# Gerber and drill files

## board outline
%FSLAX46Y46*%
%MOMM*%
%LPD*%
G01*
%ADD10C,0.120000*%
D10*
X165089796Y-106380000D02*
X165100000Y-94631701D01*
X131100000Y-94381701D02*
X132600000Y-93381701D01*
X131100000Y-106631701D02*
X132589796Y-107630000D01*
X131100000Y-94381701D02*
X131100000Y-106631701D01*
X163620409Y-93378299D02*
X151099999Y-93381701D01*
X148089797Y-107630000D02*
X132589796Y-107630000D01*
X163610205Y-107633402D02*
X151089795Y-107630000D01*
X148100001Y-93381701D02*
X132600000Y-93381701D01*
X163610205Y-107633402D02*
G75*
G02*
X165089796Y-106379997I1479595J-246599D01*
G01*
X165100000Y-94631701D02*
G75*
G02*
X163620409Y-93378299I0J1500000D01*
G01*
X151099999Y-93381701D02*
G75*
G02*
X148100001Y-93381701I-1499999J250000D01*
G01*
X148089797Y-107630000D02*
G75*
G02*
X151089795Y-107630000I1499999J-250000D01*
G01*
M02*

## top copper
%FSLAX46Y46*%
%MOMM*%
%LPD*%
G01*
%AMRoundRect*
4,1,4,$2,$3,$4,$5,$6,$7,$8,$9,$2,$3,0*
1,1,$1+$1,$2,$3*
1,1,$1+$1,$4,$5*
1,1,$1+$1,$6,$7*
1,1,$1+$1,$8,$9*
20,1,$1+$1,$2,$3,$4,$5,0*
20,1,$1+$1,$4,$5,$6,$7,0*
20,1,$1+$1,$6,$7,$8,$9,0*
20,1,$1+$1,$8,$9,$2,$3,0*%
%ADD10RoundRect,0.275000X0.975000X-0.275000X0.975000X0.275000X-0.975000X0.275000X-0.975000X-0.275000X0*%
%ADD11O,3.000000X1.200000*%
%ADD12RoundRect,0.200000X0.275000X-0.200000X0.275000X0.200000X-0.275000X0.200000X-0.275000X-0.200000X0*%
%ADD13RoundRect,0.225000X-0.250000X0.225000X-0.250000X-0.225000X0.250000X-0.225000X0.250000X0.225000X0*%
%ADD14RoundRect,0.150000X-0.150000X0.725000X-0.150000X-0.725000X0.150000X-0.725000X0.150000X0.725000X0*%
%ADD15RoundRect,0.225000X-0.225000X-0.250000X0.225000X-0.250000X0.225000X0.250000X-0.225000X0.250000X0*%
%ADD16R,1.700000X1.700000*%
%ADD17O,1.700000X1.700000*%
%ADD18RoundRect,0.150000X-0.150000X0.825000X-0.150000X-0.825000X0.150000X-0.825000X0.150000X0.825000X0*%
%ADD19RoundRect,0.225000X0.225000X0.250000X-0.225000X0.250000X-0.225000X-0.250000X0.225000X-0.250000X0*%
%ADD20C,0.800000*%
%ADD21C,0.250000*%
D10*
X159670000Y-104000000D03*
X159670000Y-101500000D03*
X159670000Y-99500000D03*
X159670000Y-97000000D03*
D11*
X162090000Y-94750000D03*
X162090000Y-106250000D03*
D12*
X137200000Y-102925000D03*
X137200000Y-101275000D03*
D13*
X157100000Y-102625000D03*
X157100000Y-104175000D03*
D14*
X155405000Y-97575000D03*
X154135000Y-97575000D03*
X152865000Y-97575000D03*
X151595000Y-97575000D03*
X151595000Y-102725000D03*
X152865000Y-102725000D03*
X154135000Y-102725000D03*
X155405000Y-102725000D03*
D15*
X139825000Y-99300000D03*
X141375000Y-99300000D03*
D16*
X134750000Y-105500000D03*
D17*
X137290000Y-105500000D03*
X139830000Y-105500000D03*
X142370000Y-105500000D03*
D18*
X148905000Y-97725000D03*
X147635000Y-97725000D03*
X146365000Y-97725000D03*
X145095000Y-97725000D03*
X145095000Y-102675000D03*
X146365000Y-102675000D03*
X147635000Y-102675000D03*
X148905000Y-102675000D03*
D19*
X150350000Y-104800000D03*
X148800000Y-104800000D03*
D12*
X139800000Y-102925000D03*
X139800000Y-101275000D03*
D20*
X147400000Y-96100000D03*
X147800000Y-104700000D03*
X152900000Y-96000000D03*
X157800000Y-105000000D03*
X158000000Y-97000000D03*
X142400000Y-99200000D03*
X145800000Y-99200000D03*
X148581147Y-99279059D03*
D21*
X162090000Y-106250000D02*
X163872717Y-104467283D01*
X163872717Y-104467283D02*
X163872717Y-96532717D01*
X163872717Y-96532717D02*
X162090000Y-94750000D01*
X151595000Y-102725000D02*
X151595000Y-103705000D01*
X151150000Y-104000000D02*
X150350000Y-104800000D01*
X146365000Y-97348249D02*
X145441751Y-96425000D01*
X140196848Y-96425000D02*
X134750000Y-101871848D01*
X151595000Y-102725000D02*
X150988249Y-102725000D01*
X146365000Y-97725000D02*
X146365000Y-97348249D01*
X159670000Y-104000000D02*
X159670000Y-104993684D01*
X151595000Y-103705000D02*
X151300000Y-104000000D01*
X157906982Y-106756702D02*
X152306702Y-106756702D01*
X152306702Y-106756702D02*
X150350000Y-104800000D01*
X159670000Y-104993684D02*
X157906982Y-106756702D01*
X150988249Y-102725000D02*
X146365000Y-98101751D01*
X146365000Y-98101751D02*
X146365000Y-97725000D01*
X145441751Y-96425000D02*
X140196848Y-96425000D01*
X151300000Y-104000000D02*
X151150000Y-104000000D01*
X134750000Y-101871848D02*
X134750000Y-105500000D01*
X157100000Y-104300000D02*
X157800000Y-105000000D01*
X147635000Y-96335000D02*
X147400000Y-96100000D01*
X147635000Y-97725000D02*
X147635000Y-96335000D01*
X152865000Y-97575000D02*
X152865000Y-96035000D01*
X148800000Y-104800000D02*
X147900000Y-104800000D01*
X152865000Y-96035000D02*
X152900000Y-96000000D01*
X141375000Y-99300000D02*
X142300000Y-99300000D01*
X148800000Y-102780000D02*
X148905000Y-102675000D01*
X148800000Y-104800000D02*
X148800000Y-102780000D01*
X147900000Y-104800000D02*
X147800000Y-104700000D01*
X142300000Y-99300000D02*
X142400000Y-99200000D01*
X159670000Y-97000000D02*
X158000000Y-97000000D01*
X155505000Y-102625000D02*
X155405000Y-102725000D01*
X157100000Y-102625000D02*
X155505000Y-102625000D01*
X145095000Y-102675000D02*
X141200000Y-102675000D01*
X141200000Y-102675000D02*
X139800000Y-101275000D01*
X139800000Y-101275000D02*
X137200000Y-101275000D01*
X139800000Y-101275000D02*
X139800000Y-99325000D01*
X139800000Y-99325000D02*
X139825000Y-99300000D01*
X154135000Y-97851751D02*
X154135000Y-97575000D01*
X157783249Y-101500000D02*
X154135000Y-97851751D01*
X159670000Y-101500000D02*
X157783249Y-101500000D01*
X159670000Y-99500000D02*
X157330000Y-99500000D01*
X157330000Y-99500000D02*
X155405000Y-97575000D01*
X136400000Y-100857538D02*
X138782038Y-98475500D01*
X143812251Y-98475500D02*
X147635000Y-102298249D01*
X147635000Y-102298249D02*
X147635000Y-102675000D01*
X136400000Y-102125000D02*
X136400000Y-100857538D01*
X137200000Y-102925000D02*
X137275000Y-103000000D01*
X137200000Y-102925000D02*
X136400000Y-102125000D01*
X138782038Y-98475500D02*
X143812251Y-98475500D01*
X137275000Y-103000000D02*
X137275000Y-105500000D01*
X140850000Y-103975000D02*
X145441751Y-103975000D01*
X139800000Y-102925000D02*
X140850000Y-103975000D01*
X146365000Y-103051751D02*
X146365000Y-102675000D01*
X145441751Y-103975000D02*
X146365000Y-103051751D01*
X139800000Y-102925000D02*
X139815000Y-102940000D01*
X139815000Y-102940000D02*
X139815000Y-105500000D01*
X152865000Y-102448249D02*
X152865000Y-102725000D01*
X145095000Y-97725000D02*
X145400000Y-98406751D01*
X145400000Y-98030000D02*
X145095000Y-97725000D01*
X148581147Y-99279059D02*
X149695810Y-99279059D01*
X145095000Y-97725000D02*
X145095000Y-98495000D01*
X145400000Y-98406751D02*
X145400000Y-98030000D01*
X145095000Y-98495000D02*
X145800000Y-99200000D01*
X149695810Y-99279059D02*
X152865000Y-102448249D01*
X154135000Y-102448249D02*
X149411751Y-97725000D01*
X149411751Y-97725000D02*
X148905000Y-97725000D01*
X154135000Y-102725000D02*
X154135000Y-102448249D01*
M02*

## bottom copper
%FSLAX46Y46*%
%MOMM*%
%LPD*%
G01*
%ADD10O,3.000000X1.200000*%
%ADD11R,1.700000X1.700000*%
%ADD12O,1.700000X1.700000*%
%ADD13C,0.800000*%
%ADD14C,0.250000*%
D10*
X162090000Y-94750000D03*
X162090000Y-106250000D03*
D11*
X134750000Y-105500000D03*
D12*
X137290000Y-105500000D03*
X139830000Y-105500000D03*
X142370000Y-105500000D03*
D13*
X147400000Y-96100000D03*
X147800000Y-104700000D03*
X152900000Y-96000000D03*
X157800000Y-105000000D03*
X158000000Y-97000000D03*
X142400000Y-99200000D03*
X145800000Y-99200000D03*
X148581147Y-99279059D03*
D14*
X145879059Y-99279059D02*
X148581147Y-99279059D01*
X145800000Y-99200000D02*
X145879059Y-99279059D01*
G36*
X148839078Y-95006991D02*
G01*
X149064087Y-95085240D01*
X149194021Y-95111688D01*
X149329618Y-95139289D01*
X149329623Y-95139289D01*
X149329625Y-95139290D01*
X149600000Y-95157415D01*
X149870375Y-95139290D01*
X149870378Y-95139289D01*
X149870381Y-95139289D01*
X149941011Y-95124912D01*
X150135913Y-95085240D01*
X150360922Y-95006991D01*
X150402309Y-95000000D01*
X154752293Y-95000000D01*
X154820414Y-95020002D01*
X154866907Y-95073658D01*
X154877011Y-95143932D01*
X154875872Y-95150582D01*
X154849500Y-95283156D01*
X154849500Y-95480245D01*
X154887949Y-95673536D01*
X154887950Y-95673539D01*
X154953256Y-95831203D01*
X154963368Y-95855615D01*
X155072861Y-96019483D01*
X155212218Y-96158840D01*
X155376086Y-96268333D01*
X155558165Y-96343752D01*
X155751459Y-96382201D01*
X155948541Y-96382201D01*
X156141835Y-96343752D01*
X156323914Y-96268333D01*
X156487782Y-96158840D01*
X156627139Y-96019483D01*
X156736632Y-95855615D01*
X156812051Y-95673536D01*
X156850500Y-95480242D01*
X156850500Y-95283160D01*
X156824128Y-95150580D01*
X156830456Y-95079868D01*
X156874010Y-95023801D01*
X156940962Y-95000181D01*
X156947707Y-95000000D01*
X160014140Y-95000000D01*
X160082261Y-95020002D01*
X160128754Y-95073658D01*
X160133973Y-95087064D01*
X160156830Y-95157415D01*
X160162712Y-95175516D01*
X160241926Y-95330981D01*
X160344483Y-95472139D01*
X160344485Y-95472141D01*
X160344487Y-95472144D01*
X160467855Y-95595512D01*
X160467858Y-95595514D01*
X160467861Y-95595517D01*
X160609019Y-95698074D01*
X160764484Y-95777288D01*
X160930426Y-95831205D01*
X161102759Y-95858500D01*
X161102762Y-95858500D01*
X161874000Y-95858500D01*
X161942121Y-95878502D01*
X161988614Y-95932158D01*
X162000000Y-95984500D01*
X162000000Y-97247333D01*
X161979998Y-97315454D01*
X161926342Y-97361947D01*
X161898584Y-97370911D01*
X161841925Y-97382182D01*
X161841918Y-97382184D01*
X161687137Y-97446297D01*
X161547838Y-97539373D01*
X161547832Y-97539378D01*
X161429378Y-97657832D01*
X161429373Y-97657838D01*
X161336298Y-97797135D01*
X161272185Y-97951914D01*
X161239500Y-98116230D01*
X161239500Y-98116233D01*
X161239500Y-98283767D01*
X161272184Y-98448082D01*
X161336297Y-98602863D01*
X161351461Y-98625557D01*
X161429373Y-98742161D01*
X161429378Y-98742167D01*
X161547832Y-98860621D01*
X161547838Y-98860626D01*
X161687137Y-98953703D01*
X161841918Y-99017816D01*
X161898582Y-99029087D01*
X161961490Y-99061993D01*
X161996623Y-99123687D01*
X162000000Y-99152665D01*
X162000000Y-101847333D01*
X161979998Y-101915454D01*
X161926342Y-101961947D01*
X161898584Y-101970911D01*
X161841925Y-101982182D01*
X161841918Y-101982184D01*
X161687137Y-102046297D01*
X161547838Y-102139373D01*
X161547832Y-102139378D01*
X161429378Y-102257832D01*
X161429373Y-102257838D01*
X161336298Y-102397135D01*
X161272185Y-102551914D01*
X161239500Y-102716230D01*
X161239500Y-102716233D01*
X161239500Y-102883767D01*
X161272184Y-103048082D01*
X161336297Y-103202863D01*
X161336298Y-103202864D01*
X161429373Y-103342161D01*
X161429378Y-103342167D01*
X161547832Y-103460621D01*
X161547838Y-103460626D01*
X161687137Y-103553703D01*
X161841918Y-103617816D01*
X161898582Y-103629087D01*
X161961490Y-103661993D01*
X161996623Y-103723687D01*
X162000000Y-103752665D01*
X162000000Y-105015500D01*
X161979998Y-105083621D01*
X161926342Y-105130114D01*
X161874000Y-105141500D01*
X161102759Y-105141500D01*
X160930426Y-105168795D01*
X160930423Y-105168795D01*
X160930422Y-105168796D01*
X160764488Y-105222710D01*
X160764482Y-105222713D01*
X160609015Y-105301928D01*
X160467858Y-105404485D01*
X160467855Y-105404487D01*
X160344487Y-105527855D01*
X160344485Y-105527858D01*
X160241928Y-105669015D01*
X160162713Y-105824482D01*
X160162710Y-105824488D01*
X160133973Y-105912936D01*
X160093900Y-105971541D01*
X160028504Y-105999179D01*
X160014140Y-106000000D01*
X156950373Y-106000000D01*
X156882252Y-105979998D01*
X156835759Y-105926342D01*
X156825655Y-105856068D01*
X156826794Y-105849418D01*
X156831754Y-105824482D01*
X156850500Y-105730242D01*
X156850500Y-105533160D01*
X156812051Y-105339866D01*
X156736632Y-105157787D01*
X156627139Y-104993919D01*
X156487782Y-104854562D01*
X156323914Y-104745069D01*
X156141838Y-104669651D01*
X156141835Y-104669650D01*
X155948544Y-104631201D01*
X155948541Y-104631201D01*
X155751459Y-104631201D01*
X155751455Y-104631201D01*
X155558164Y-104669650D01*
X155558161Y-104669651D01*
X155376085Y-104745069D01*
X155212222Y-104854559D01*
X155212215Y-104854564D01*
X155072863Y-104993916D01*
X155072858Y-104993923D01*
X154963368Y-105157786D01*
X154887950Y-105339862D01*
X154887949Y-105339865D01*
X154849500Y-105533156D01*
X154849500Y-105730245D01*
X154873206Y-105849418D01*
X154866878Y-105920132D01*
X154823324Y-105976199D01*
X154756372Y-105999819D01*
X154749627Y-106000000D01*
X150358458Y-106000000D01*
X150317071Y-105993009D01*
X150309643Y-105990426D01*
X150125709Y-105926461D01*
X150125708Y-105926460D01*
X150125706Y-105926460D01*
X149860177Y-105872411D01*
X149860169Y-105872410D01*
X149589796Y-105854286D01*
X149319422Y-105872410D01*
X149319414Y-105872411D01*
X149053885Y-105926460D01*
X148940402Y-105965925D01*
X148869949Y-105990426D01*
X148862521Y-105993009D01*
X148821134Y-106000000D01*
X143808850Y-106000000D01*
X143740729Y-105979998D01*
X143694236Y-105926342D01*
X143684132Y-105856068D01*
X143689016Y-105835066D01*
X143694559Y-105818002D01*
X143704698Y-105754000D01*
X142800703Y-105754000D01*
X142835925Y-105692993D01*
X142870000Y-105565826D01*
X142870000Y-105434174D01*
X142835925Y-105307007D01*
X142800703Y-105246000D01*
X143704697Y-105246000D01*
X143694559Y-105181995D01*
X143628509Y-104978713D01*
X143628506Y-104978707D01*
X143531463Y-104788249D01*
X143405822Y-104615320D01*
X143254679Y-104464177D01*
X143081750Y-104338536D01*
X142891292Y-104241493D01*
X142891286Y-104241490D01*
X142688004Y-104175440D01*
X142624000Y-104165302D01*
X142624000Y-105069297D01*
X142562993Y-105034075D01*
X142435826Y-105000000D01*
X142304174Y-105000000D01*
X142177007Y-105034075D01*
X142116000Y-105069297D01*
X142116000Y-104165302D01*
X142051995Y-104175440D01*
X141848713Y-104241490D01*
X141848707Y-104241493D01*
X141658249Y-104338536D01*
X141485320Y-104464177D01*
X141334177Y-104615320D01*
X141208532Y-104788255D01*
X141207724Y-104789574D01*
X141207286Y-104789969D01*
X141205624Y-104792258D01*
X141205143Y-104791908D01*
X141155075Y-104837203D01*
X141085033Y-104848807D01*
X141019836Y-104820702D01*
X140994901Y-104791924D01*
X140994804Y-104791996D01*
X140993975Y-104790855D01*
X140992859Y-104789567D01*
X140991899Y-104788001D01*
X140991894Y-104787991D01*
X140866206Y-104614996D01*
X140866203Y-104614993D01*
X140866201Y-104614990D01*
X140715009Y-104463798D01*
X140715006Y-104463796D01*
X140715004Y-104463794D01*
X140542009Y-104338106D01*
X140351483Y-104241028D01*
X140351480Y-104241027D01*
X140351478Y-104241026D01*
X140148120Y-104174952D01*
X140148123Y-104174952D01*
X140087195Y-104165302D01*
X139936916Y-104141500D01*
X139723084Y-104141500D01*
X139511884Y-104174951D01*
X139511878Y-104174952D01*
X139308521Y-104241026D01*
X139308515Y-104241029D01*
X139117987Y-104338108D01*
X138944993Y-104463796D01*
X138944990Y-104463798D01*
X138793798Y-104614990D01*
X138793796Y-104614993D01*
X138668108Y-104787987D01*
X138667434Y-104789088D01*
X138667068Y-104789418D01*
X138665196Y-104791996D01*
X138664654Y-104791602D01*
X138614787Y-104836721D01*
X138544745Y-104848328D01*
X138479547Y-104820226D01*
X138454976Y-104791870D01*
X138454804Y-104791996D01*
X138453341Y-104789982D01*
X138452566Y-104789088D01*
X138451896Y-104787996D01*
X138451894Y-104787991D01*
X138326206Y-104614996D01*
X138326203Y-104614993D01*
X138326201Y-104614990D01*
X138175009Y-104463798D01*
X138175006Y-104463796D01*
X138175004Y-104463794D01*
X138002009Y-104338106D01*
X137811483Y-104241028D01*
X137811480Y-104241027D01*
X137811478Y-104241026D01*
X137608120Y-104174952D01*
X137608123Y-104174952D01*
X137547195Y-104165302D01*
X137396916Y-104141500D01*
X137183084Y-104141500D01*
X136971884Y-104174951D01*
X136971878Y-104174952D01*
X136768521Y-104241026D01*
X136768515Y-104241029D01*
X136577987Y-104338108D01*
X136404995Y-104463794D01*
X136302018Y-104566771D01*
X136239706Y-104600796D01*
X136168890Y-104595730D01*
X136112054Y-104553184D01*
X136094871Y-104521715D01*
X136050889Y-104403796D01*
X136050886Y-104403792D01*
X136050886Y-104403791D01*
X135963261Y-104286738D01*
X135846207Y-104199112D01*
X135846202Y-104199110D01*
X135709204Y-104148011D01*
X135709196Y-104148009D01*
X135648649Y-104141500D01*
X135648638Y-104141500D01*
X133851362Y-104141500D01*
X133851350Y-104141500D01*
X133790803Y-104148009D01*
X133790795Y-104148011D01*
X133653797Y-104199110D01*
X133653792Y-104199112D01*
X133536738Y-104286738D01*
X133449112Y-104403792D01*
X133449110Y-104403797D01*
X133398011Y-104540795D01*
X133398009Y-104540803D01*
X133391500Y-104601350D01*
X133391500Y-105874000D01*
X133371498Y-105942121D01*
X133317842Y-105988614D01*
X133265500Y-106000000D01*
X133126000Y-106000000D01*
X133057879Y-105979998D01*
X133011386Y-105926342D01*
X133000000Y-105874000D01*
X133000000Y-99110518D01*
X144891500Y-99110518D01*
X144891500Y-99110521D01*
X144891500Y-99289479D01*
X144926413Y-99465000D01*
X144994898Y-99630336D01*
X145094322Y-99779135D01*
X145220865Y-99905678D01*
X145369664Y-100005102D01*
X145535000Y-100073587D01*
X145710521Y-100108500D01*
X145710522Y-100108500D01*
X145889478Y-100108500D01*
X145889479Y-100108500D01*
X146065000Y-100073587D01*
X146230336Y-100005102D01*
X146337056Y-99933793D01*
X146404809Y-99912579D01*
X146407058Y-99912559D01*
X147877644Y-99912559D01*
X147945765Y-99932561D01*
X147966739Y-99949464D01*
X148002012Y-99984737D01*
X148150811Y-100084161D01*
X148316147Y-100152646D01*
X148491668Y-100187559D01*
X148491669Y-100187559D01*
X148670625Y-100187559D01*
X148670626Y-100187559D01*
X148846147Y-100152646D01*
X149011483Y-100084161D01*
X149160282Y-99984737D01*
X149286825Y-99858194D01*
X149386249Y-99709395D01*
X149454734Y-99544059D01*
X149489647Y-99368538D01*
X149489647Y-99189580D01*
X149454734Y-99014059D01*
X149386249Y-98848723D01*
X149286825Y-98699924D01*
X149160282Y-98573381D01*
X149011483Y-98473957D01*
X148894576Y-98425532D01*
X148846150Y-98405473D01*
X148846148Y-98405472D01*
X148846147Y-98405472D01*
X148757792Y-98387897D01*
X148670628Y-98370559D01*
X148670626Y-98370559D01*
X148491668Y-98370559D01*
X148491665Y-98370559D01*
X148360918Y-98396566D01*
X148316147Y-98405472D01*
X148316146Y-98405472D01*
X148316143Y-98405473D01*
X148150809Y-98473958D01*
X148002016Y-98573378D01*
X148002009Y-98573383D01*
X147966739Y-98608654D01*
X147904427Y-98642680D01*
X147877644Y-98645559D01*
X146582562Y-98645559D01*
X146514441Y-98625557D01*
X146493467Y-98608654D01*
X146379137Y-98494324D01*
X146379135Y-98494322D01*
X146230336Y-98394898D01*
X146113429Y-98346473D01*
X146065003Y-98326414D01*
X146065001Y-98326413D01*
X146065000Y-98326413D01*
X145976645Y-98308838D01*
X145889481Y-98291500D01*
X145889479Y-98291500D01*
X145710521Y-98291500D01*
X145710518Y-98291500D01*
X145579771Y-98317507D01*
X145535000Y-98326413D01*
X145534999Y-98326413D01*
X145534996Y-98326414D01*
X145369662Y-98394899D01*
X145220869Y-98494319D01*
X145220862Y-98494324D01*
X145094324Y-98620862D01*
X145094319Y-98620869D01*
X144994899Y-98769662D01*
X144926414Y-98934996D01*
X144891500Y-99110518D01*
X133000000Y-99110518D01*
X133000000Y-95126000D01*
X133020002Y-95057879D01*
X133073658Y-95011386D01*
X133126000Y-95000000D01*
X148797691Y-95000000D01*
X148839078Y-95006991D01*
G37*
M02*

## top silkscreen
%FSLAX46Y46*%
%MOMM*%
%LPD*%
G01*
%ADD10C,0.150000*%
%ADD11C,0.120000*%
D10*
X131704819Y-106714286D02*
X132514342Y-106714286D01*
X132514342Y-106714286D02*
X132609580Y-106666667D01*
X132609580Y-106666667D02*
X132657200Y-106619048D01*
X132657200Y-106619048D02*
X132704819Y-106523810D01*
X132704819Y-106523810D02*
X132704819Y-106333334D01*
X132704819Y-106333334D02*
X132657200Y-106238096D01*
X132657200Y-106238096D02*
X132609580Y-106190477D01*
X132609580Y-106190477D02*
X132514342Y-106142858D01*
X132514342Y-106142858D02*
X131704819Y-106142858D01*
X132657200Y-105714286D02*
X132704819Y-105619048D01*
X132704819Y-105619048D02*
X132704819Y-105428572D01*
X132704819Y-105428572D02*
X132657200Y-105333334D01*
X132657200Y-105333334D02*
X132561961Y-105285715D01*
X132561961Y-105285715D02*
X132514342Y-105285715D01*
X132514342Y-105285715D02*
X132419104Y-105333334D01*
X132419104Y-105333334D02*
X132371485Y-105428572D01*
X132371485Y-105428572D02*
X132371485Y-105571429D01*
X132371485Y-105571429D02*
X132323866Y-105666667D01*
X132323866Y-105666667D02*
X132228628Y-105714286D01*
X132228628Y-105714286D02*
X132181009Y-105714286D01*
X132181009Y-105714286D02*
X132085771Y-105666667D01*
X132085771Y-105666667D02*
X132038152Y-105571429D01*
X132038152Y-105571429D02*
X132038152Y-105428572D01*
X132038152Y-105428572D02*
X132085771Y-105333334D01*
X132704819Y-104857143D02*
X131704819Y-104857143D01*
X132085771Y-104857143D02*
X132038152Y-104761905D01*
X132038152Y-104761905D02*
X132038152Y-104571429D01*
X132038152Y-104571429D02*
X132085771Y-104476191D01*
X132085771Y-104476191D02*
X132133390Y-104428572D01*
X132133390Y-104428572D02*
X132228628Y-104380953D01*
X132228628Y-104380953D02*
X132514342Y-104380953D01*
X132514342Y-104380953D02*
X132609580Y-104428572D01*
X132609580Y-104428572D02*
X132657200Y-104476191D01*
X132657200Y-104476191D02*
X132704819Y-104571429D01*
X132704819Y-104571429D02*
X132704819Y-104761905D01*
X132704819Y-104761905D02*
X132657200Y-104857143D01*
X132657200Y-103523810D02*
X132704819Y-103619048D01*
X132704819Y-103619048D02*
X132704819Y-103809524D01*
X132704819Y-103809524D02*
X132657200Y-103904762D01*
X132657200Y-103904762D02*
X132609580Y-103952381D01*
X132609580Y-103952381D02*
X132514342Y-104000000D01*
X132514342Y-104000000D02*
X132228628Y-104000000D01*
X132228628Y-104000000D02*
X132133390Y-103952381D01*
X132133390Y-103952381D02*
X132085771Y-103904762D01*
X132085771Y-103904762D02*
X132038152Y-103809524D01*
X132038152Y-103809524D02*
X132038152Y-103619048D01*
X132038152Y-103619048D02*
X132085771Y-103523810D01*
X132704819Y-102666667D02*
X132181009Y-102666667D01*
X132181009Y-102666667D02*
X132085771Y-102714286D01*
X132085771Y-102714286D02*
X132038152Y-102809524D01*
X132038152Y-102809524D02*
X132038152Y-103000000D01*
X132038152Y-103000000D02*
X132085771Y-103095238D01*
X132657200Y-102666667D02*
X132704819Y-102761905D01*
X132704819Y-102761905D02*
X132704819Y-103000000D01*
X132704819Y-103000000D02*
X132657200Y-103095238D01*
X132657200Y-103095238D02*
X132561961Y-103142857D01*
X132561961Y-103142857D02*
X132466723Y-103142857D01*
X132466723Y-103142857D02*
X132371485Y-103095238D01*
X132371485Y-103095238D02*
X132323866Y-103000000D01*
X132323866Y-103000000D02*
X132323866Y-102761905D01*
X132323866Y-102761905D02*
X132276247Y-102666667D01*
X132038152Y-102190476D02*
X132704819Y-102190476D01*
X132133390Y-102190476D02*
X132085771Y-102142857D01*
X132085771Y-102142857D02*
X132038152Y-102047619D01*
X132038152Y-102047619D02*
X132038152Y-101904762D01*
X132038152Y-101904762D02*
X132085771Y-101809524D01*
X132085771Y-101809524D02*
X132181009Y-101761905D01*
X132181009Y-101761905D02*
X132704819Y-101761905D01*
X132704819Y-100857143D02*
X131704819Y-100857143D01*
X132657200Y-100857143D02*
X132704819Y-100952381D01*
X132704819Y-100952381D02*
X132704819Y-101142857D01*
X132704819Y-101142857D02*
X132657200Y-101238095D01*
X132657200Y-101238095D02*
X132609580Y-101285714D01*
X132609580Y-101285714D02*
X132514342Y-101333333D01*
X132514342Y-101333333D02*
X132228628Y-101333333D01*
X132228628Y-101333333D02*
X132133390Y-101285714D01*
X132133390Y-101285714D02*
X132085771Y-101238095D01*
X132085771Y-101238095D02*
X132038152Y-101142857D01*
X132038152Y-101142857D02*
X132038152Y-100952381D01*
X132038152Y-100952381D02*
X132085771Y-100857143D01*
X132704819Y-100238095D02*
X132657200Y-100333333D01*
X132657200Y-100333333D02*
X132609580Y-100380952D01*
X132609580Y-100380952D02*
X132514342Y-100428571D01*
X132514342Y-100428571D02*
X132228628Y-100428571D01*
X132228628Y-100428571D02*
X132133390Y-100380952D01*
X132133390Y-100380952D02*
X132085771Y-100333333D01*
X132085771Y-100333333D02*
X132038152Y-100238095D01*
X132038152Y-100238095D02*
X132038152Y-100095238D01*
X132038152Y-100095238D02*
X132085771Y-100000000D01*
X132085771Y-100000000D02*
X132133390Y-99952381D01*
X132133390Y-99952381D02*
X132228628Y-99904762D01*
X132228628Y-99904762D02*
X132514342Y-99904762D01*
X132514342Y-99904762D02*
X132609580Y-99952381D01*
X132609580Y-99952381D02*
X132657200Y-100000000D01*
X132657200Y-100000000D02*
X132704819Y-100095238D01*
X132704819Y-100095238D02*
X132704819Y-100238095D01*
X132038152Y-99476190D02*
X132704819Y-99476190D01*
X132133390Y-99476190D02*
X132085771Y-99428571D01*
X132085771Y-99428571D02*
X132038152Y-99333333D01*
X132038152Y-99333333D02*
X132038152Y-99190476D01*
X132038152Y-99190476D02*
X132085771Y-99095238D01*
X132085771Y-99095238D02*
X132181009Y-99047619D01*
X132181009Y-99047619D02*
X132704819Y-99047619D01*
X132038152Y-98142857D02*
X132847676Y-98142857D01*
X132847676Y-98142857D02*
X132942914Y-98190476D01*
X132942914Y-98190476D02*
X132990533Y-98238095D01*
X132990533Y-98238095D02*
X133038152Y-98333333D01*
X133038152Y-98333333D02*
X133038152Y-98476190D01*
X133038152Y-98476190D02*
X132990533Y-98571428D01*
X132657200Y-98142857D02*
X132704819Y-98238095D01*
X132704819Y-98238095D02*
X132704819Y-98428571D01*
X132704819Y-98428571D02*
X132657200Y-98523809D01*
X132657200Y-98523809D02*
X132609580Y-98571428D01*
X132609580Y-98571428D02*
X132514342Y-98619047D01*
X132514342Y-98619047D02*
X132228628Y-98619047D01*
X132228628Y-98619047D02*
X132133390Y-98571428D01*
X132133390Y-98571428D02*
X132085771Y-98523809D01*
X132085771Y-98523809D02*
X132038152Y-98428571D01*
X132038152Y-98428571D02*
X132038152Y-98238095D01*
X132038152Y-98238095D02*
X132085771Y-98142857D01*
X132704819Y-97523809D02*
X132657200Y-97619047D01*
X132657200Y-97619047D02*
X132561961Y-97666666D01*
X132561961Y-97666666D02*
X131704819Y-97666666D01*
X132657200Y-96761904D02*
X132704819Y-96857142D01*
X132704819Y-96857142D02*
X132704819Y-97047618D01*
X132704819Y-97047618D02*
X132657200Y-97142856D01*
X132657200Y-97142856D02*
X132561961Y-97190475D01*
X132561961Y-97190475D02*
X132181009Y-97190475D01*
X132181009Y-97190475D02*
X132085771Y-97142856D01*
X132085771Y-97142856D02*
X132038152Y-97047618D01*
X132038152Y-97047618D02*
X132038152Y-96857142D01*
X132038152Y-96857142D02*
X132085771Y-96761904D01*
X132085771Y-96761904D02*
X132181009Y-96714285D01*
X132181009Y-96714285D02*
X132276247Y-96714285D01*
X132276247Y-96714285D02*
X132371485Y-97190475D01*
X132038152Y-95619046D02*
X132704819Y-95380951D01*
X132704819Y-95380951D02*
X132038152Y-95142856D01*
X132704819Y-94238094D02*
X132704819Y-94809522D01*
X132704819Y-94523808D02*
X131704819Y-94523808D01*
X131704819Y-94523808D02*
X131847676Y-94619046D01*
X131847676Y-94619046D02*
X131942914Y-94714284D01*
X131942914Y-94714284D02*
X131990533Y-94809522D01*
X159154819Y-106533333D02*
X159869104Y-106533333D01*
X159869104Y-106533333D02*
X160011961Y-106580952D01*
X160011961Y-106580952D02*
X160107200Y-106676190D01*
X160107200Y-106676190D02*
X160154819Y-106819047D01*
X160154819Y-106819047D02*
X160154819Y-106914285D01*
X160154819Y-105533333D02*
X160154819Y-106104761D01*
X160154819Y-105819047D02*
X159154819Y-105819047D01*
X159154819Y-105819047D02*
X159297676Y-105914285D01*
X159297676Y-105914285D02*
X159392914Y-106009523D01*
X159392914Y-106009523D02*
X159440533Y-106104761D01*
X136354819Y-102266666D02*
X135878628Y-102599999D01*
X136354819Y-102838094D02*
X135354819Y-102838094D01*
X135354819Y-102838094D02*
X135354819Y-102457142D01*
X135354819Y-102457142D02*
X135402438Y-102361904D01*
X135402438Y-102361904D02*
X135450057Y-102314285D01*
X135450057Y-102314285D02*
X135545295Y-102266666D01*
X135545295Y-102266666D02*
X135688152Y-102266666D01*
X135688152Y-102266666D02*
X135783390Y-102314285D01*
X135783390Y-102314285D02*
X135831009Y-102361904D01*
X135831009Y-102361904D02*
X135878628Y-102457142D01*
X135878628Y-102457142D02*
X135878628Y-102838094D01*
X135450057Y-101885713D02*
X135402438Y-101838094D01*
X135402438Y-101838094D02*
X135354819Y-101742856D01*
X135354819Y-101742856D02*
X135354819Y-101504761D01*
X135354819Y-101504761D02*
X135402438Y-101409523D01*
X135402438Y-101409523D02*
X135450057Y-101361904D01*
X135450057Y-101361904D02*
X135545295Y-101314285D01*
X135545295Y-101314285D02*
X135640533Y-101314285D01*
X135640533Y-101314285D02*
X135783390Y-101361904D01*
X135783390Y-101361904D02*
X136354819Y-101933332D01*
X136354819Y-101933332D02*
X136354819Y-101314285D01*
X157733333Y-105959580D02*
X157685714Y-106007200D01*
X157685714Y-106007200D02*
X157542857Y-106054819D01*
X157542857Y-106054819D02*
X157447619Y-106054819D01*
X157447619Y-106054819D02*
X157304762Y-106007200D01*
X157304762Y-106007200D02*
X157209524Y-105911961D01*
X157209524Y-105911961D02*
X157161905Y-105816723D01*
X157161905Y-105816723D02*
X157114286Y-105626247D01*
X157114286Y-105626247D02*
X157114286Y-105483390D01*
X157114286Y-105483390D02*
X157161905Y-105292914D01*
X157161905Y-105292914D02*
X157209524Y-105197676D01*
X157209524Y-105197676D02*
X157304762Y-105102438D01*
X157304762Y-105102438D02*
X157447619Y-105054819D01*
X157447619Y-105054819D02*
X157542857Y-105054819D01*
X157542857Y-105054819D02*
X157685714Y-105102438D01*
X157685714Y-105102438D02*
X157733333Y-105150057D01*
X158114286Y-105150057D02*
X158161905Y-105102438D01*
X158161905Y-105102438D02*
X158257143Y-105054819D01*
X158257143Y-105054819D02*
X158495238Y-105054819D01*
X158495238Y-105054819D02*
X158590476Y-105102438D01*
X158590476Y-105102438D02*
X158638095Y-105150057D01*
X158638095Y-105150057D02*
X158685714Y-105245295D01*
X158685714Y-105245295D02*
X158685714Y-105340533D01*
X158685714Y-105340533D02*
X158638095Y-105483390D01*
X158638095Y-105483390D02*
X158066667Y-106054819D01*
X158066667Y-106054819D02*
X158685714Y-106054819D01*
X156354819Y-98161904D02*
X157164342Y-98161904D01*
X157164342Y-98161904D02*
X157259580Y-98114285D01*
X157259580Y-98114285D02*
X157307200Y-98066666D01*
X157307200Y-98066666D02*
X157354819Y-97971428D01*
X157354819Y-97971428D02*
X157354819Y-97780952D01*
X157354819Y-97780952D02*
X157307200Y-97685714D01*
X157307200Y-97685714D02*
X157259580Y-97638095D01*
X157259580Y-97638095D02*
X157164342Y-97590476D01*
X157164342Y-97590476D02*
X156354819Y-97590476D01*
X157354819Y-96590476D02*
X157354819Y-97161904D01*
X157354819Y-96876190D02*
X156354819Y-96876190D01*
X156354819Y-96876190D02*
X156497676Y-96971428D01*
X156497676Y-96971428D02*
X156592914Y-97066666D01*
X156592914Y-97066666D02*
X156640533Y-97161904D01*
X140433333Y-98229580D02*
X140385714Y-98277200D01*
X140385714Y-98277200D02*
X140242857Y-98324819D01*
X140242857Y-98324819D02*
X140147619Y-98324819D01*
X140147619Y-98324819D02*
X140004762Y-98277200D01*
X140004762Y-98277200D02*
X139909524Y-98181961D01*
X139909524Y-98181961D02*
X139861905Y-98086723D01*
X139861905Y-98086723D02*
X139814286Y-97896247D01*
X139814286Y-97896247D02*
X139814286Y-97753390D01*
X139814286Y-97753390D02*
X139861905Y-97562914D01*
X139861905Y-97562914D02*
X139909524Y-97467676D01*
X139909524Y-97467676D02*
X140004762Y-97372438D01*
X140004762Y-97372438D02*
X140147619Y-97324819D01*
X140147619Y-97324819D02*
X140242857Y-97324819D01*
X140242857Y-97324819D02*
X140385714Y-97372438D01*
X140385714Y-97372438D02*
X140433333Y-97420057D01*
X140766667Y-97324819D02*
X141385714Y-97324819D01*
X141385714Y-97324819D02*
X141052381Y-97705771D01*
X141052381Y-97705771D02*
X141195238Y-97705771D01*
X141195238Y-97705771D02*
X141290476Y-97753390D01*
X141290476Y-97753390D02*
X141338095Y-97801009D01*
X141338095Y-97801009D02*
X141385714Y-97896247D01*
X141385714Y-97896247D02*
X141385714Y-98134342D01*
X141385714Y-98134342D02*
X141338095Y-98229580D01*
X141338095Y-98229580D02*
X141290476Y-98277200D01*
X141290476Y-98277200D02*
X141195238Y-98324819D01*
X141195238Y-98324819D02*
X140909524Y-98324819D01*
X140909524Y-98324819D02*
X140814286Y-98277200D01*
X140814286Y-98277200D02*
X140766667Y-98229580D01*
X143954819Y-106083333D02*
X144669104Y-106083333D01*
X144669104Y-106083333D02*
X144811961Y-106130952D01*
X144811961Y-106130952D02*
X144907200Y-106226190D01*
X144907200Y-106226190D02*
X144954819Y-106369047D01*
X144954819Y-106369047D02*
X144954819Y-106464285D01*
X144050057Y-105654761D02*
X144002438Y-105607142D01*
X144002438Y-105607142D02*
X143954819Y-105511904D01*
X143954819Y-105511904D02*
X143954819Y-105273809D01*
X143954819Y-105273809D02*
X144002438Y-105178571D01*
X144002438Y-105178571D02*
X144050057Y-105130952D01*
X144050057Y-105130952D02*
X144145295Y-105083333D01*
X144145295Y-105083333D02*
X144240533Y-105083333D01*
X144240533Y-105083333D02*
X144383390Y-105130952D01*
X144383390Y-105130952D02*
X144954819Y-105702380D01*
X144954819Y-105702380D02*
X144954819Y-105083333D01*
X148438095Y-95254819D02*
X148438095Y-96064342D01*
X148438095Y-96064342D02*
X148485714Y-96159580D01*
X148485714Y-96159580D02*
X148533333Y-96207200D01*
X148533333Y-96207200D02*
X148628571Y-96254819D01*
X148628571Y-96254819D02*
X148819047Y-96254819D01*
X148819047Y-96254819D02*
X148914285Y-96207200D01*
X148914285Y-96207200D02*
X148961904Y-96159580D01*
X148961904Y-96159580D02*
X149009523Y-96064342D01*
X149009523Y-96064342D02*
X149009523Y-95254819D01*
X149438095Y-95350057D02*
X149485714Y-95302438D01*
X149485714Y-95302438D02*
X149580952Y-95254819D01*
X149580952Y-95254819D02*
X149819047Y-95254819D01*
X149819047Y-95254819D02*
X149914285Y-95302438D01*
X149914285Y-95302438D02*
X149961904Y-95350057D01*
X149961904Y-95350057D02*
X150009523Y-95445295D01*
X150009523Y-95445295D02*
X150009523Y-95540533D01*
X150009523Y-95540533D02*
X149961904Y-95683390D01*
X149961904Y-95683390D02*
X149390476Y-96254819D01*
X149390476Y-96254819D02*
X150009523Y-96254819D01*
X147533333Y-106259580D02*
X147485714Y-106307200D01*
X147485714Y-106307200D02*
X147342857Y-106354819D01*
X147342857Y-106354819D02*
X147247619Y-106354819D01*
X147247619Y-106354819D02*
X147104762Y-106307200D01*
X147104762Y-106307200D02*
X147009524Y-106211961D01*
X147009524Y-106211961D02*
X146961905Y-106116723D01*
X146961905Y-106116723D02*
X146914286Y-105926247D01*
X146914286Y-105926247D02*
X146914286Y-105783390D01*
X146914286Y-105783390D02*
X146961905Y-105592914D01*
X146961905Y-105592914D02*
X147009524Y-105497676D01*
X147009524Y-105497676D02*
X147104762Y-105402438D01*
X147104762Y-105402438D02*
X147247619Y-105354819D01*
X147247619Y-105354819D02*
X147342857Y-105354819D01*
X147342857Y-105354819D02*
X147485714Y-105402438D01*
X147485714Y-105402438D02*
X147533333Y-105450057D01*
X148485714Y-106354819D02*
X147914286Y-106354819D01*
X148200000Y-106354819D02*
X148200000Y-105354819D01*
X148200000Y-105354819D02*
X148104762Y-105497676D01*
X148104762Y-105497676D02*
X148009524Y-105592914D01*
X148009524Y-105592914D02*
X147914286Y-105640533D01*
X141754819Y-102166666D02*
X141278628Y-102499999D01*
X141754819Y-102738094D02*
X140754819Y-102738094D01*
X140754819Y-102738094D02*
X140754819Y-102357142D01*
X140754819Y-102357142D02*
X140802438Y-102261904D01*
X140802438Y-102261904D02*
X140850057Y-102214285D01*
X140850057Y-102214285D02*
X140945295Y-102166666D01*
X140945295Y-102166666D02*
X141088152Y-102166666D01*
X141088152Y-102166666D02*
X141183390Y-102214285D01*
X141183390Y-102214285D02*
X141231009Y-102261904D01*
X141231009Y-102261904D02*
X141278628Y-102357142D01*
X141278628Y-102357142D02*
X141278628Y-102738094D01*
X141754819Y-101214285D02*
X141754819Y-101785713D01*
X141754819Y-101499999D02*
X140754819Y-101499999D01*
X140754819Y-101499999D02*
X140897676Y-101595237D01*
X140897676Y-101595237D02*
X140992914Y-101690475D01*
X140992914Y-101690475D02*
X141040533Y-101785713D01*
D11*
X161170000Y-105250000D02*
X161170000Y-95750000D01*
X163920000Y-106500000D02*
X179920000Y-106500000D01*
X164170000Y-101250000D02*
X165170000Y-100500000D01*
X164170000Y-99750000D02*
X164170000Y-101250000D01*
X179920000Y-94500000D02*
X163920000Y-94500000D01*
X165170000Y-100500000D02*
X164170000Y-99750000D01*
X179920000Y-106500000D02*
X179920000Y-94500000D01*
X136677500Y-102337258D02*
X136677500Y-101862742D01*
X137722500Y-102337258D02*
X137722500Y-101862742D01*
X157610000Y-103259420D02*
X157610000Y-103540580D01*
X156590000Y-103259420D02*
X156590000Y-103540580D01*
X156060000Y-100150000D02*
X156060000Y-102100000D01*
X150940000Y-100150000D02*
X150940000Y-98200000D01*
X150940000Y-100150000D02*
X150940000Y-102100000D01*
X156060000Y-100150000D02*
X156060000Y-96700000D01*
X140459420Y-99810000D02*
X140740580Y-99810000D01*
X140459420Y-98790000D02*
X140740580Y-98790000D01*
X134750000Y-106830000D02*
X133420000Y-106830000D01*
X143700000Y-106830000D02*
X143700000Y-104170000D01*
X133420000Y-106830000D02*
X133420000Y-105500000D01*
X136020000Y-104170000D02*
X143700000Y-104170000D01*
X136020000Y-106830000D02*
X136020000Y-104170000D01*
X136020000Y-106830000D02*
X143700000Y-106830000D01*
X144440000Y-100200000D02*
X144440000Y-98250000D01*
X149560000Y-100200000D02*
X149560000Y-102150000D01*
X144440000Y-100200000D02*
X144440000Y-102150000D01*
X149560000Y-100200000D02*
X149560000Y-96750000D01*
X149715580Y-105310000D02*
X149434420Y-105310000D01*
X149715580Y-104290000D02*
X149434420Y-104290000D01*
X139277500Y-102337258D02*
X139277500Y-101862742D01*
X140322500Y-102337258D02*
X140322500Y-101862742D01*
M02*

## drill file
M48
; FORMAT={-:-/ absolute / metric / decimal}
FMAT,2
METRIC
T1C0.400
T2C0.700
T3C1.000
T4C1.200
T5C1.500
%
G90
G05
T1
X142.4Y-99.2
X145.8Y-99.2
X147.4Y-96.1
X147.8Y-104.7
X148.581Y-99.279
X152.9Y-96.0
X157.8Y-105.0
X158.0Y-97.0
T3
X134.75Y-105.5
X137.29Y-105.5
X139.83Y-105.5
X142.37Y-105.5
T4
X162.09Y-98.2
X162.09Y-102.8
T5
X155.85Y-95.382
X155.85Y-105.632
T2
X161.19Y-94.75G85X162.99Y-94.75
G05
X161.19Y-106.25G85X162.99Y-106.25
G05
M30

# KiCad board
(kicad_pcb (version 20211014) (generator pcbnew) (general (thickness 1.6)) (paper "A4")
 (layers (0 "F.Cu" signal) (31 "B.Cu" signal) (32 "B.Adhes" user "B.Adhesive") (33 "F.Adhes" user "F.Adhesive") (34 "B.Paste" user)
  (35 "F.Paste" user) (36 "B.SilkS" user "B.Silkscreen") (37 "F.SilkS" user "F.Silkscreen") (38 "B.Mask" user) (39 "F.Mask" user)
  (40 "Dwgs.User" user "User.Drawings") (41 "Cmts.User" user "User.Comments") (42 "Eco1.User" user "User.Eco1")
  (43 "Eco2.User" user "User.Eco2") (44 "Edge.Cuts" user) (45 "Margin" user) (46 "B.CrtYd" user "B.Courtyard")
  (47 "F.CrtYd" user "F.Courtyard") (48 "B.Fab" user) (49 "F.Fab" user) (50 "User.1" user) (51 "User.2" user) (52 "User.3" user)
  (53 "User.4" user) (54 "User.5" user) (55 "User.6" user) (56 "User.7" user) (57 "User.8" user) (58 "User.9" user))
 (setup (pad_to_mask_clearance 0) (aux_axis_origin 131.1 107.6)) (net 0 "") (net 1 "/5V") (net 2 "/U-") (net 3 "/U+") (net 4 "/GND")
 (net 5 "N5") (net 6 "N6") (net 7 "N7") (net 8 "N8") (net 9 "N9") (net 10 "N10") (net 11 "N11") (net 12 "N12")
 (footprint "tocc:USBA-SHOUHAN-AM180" (layer "F.Cu") (at 159.67 100.5 90)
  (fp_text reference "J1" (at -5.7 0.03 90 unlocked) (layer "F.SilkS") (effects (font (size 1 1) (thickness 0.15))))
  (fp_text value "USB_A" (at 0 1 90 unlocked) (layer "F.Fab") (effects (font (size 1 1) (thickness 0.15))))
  (fp_line (start -4.75 1.5) (end 4.75 1.5) (layer "F.SilkS") (width 0.12))
  (fp_line (start -6 4.25) (end -6 20.25) (layer "F.SilkS") (width 0.12))
  (fp_line (start -0.75 4.5) (end 0 5.5) (layer "F.SilkS") (width 0.12))
  (fp_line (start 0.75 4.5) (end -0.75 4.5) (layer "F.SilkS") (width 0.12))
  (fp_line (start 6 20.25) (end 6 4.25) (layer "F.SilkS") (width 0.12))
  (fp_line (start 0 5.5) (end 0.75 4.5) (layer "F.SilkS") (width 0.12))
  (fp_line (start -6 20.25) (end 6 20.25) (layer "F.SilkS") (width 0.12))
  (pad "" np_thru_hole circle (at -2.3 2.42 90) (size 1.2 1.2) (drill 1.2) (layers F&B.Cu *.Mask))
  (pad "" np_thru_hole circle (at 2.3 2.42 90) (size 1.2 1.2) (drill 1.2) (layers F&B.Cu *.Mask))
  (pad "1" smd roundrect (at -3.5 0 90) (size 1.1 2.5) (layers "F.Cu" "F.Paste" "F.Mask") (roundrect_rratio 0.25) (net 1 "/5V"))
  (pad "2" smd roundrect (at -1 0 90) (size 1.1 2.5) (layers "F.Cu" "F.Paste" "F.Mask") (roundrect_rratio 0.25) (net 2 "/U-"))
  (pad "3" smd roundrect (at 1 0 90) (size 1.1 2.5) (layers "F.Cu" "F.Paste" "F.Mask") (roundrect_rratio 0.25) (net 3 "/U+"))
  (pad "4" smd roundrect (at 3.5 0 90) (size 1.1 2.5) (layers "F.Cu" "F.Paste" "F.Mask") (roundrect_rratio 0.25) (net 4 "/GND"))
  (pad "5" thru_hole oval (at 5.75 2.42 90) (size 1.2 3) (drill oval 0.7 2.5) (layers *.Cu *.Mask) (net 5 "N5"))
  (pad "5" thru_hole oval (at -5.75 2.42 90) (size 1.2 3) (drill oval 0.7 2.5) (layers *.Cu *.Mask) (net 5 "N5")))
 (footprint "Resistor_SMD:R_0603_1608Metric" (layer "F.Cu") (at 137.2 102.1 90)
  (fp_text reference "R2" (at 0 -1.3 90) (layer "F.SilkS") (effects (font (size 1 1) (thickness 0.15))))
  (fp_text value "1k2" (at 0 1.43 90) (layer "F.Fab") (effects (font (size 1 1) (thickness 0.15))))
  (fp_line (start -0.237258 -0.5225) (end 0.237258 -0.5225) (layer "F.SilkS") (width 0.12))
  (fp_line (start -0.237258 0.5225) (end 0.237258 0.5225) (layer "F.SilkS") (width 0.12))
  (pad "1" smd roundrect (at -0.825 0 90) (size 0.8 0.95) (layers "F.Cu" "F.Paste" "F.Mask") (roundrect_rratio 0.25) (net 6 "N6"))
  (pad "2" smd roundrect (at 0.825 0 90) (size 0.8 0.95) (layers "F.Cu" "F.Paste" "F.Mask") (roundrect_rratio 0.25) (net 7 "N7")))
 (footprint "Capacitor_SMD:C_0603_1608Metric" (layer "F.Cu") (at 157.1 103.4 -90)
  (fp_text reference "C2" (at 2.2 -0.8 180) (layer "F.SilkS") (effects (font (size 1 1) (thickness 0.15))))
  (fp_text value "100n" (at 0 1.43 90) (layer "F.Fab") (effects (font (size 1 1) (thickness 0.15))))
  (fp_line (start -0.14058 -0.51) (end 0.14058 -0.51) (layer "F.SilkS") (width 0.12))
  (fp_line (start -0.14058 0.51) (end 0.14058 0.51) (layer "F.SilkS") (width 0.12))
  (pad "1" smd roundrect (at -0.775 0 270) (size 0.9 0.95) (layers "F.Cu" "F.Paste" "F.Mask") (roundrect_rratio 0.25) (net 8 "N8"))
  (pad "2" smd roundrect (at 0.775 0 270) (size 0.9 0.95) (layers "F.Cu" "F.Paste" "F.Mask") (roundrect_rratio 0.25) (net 4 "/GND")))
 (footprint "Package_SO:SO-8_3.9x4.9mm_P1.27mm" (layer "F.Cu") (at 153.5 100.15 -90)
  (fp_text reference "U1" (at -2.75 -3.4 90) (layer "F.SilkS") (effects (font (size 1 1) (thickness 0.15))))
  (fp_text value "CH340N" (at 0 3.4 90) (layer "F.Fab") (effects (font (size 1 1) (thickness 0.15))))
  (fp_line (start 0 -2.56) (end 1.95 -2.56) (layer "F.SilkS") (width 0.12))
  (fp_line (start 0 2.56) (end -1.95 2.56) (layer "F.SilkS") (width 0.12))
  (fp_line (start 0 2.56) (end 1.95 2.56) (layer "F.SilkS") (width 0.12))
  (fp_line (start 0 -2.56) (end -3.45 -2.56) (layer "F.SilkS") (width 0.12))
  (pad "1" smd roundrect (at -2.575 -1.905 270) (size 1.75 0.6) (layers "F.Cu" "F.Paste" "F.Mask") (roundrect_rratio 0.25) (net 3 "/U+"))
  (pad "2" smd roundrect (at -2.575 -0.635 270) (size 1.75 0.6) (layers "F.Cu" "F.Paste" "F.Mask") (roundrect_rratio 0.25) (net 2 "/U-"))
  (pad "3" smd roundrect (at -2.575 0.635 270) (size 1.75 0.6) (layers "F.Cu" "F.Paste" "F.Mask") (roundrect_rratio 0.25) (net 4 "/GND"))
  (pad "4" smd roundrect (at -2.575 1.905 270) (size 1.75 0.6) (layers "F.Cu" "F.Paste" "F.Mask") (roundrect_rratio 0.25) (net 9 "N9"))
  (pad "5" smd roundrect (at 2.575 1.905 270) (size 1.75 0.6) (layers "F.Cu" "F.Paste" "F.Mask") (roundrect_rratio 0.25) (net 1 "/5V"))
  (pad "6" smd roundrect (at 2.575 0.635 270) (size 1.75 0.6) (layers "F.Cu" "F.Paste" "F.Mask") (roundrect_rratio 0.25) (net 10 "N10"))
  (pad "7" smd roundrect (at 2.575 -0.635 270) (size 1.75 0.6) (layers "F.Cu" "F.Paste" "F.Mask") (roundrect_rratio 0.25) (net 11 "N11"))
  (pad "8" smd roundrect (at 2.575 -1.905 270) (size 1.75 0.6) (layers "F.Cu" "F.Paste" "F.Mask") (roundrect_rratio 0.25) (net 8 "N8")))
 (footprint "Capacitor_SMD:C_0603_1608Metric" (layer "F.Cu") (at 140.6 99.3)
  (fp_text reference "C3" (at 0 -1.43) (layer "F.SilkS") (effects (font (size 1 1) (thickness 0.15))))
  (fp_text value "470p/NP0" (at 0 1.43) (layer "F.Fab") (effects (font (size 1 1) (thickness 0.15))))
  (fp_line (start -0.14058 0.51) (end 0.14058 0.51) (layer "F.SilkS") (width 0.12))
  (fp_line (start -0.14058 -0.51) (end 0.14058 -0.51) (layer "F.SilkS") (width 0.12))
  (pad "1" smd roundrect (at -0.775 0) (size 0.9 0.95) (layers "F.Cu" "F.Paste" "F.Mask") (roundrect_rratio 0.25) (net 7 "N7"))
  (pad "2" smd roundrect (at 0.775 0) (size 0.9 0.95) (layers "F.Cu" "F.Paste" "F.Mask") (roundrect_rratio 0.25) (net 4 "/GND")))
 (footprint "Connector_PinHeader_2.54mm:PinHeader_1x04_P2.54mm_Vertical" (layer "F.Cu") (at 134.75 105.5 90)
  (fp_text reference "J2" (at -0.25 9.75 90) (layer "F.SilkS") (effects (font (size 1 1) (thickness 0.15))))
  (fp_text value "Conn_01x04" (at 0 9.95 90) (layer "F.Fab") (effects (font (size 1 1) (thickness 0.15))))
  (fp_line (start -1.33 0) (end -1.33 -1.33) (layer "F.SilkS") (width 0.12))
  (fp_line (start -1.33 8.95) (end 1.33 8.95) (layer "F.SilkS") (width 0.12))
  (fp_line (start -1.33 -1.33) (end 0 -1.33) (layer "F.SilkS") (width 0.12))
  (fp_line (start 1.33 1.27) (end 1.33 8.95) (layer "F.SilkS") (width 0.12))
  (fp_line (start -1.33 1.27) (end 1.33 1.27) (layer "F.SilkS") (width 0.12))
  (fp_line (start -1.33 1.27) (end -1.33 8.95) (layer "F.SilkS") (width 0.12))
  (pad "1" thru_hole rect (at 0 0 90) (size 1.7 1.7) (drill 1) (layers *.Cu *.Mask) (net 1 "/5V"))
  (pad "2" thru_hole oval (at 0 2.54 90) (size 1.7 1.7) (drill 1) (layers *.Cu *.Mask) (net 6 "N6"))
  (pad "3" thru_hole oval (at 0 5.08 90) (size 1.7 1.7) (drill 1) (layers *.Cu *.Mask) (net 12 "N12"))
  (pad "4" thru_hole oval (at 0 7.62 90) (size 1.7 1.7) (drill 1) (layers *.Cu *.Mask) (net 4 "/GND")))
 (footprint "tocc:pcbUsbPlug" (layer "F.Cu") (at 129.1 107.631701)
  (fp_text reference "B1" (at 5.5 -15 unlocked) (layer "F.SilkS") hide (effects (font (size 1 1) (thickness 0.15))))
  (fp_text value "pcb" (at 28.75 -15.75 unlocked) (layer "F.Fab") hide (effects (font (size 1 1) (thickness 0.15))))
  (fp_line (start 35.989796 -1.251701) (end 36 -13) (layer "Edge.Cuts") (width 0.12))
  (fp_line (start 2 -13.25) (end 3.5 -14.25) (layer "Edge.Cuts") (width 0.12))
  (fp_line (start 2 -1) (end 3.489796 -0.001701) (layer "Edge.Cuts") (width 0.12))
  (fp_line (start 2 -13.25) (end 2 -1) (layer "Edge.Cuts") (width 0.12))
  (fp_line (start 34.520409 -14.253402) (end 21.999999 -14.25) (layer "Edge.Cuts") (width 0.12))
  (fp_line (start 18.989797 -0.001701) (end 3.489796 -0.001701) (layer "Edge.Cuts") (width 0.12))
  (fp_line (start 34.510205 0.001701) (end 21.989795 -0.001701) (layer "Edge.Cuts") (width 0.12))
  (fp_line (start 19.000001 -14.25) (end 3.5 -14.25) (layer "Edge.Cuts") (width 0.12))
  (fp_arc (start 34.510205 0.001701) (mid 35.020233 -0.896232) (end 35.989796 -1.251701) (layer "Edge.Cuts") (width 0.12))
  (fp_arc (start 36 -13) (mid 35.030437 -13.35547) (end 34.520409 -14.253402) (layer "Edge.Cuts") (width 0.12))
  (fp_arc (start 21.999999 -14.25) (mid 20.5 -12.97931) (end 19.000001 -14.25) (layer "Edge.Cuts") (width 0.12))
  (fp_arc (start 18.989797 -0.001701) (mid 20.489796 -1.272391) (end 21.989795 -0.001701) (layer "Edge.Cuts") (width 0.12))
  (pad "" np_thru_hole circle (at 26.75 -12.25) (size 1.5 1.5) (drill 1.5) (layers F&B.Cu *.Mask))
  (pad "" np_thru_hole circle (at 26.75 -2) (size 1.5 1.5) (drill 1.5) (layers F&B.Cu *.Mask)))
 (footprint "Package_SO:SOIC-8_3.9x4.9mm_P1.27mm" (layer "F.Cu") (at 147 100.2 -90)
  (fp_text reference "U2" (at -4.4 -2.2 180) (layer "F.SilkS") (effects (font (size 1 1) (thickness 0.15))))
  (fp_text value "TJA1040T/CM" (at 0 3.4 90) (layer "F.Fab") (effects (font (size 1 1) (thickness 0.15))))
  (fp_line (start 0 2.56) (end -1.95 2.56) (layer "F.SilkS") (width 0.12))
  (fp_line (start 0 -2.56) (end 1.95 -2.56) (layer "F.SilkS") (width 0.12))
  (fp_line (start 0 2.56) (end 1.95 2.56) (layer "F.SilkS") (width 0.12))
  (fp_line (start 0 -2.56) (end -3.45 -2.56) (layer "F.SilkS") (width 0.12))
  (pad "1" smd roundrect (at -2.475 -1.905 270) (size 1.95 0.6) (layers "F.Cu" "F.Paste" "F.Mask") (roundrect_rratio 0.25) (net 11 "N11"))
  (pad "2" smd roundrect (at -2.475 -0.635 270) (size 1.95 0.6) (layers "F.Cu" "F.Paste" "F.Mask") (roundrect_rratio 0.25) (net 4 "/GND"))
  (pad "3" smd roundrect (at -2.475 0.635 270) (size 1.95 0.6) (layers "F.Cu" "F.Paste" "F.Mask") (roundrect_rratio 0.25) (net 1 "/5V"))
  (pad "4" smd roundrect (at -2.475 1.905 270) (size 1.95 0.6) (layers "F.Cu" "F.Paste" "F.Mask") (roundrect_rratio 0.25) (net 10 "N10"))
  (pad "5" smd roundrect (at 2.475 1.905 270) (size 1.95 0.6) (layers "F.Cu" "F.Paste" "F.Mask") (roundrect_rratio 0.25) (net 7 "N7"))
  (pad "6" smd roundrect (at 2.475 0.635 270) (size 1.95 0.6) (layers "F.Cu" "F.Paste" "F.Mask") (roundrect_rratio 0.25) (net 12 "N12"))
  (pad "7" smd roundrect (at 2.475 -0.635 270) (size 1.95 0.6) (layers "F.Cu" "F.Paste" "F.Mask") (roundrect_rratio 0.25) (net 6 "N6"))
  (pad "8" smd roundrect (at 2.475 -1.905 270) (size 1.95 0.6) (layers "F.Cu" "F.Paste" "F.Mask") (roundrect_rratio 0.25) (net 4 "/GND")))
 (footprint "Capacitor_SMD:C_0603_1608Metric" (layer "F.Cu") (at 149.575 104.8 180)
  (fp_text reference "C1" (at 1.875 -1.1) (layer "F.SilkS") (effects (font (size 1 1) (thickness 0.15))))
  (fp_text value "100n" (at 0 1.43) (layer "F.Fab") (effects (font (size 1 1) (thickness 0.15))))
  (fp_line (start -0.14058 -0.51) (end 0.14058 -0.51) (layer "F.SilkS") (width 0.12))
  (fp_line (start -0.14058 0.51) (end 0.14058 0.51) (layer "F.SilkS") (width 0.12))
  (pad "1" smd roundrect (at -0.775 0 180) (size 0.9 0.95) (layers "F.Cu" "F.Paste" "F.Mask") (roundrect_rratio 0.25) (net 1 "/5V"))
  (pad "2" smd roundrect (at 0.775 0 180) (size 0.9 0.95) (layers "F.Cu" "F.Paste" "F.Mask") (roundrect_rratio 0.25) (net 4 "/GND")))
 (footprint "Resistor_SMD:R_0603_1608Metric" (layer "F.Cu") (at 139.8 102.1 90)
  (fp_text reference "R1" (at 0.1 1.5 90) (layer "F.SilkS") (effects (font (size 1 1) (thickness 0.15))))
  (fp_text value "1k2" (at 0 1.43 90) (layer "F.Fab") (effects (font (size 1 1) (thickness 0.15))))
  (fp_line (start -0.237258 -0.5225) (end 0.237258 -0.5225) (layer "F.SilkS") (width 0.12))
  (fp_line (start -0.237258 0.5225) (end 0.237258 0.5225) (layer "F.SilkS") (width 0.12))
  (pad "1" smd roundrect (at -0.825 0 90) (size 0.8 0.95) (layers "F.Cu" "F.Paste" "F.Mask") (roundrect_rratio 0.25) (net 12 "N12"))
  (pad "2" smd roundrect (at 0.825 0 90) (size 0.8 0.95) (layers "F.Cu" "F.Paste" "F.Mask") (roundrect_rratio 0.25) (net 7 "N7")))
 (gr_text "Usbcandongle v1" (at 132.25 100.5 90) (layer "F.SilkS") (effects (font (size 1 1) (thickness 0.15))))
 (segment (start 162.09 106.25) (end 163.872717 104.467283) (width 0.25) (layer "F.Cu") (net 5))
 (segment (start 163.872717 104.467283) (end 163.872717 96.532717) (width 0.25) (layer "F.Cu") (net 5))
 (segment (start 163.872717 96.532717) (end 162.09 94.75) (width 0.25) (layer "F.Cu") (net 5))
 (segment (start 151.595 102.725) (end 151.595 103.705) (width 0.25) (layer "F.Cu") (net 1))
 (segment (start 151.15 104) (end 150.35 104.8) (width 0.25) (layer "F.Cu") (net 1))
 (segment (start 146.365 97.348249) (end 145.441751 96.425) (width 0.25) (layer "F.Cu") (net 1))
 (segment (start 140.196848 96.425) (end 134.75 101.871848) (width 0.25) (layer "F.Cu") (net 1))
 (segment (start 151.595 102.725) (end 150.988249 102.725) (width 0.25) (layer "F.Cu") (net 1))
 (segment (start 146.365 97.725) (end 146.365 97.348249) (width 0.25) (layer "F.Cu") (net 1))
 (segment (start 159.67 104) (end 159.67 104.993684) (width 0.25) (layer "F.Cu") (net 1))
 (segment (start 151.595 103.705) (end 151.3 104) (width 0.25) (layer "F.Cu") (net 1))
 (segment (start 157.906982 106.756702) (end 152.306702 106.756702) (width 0.25) (layer "F.Cu") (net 1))
 (segment (start 152.306702 106.756702) (end 150.35 104.8) (width 0.25) (layer "F.Cu") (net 1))
 (segment (start 159.67 104.993684) (end 157.906982 106.756702) (width 0.25) (layer "F.Cu") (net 1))
 (segment (start 150.988249 102.725) (end 146.365 98.101751) (width 0.25) (layer "F.Cu") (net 1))
 (segment (start 146.365 98.101751) (end 146.365 97.725) (width 0.25) (layer "F.Cu") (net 1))
 (segment (start 145.441751 96.425) (end 140.196848 96.425) (width 0.25) (layer "F.Cu") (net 1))
 (segment (start 151.3 104) (end 151.15 104) (width 0.25) (layer "F.Cu") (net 1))
 (segment (start 134.75 101.871848) (end 134.75 105.5) (width 0.25) (layer "F.Cu") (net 1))
 (segment (start 157.1 104.3) (end 157.8 105) (width 0.25) (layer "F.Cu") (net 4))
 (segment (start 147.635 96.335) (end 147.4 96.1) (width 0.25) (layer "F.Cu") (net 4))
 (segment (start 147.635 97.725) (end 147.635 96.335) (width 0.25) (layer "F.Cu") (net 4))
 (segment (start 152.865 97.575) (end 152.865 96.035) (width 0.25) (layer "F.Cu") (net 4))
 (segment (start 148.8 104.8) (end 147.9 104.8) (width 0.25) (layer "F.Cu") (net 4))
 (segment (start 152.865 96.035) (end 152.9 96) (width 0.25) (layer "F.Cu") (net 4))
 (segment (start 141.375 99.3) (end 142.3 99.3) (width 0.25) (layer "F.Cu") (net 4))
 (segment (start 148.8 102.78) (end 148.905 102.675) (width 0.25) (layer "F.Cu") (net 4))
 (segment (start 148.8 104.8) (end 148.8 102.78) (width 0.25) (layer "F.Cu") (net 4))
 (segment (start 147.9 104.8) (end 147.8 104.7) (width 0.25) (layer "F.Cu") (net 4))
 (segment (start 142.3 99.3) (end 142.4 99.2) (width 0.25) (layer "F.Cu") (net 4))
 (segment (start 159.67 97) (end 158 97) (width 0.25) (layer "F.Cu") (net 4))
 (via (at 147.4 96.1) (size 0.8) (drill 0.4) (layers "F.Cu" "B.Cu") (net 4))
 (via (at 147.8 104.7) (size 0.8) (drill 0.4) (layers "F.Cu" "B.Cu") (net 4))
 (via (at 152.9 96) (size 0.8) (drill 0.4) (layers "F.Cu" "B.Cu") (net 4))
 (via (at 157.8 105) (size 0.8) (drill 0.4) (layers "F.Cu" "B.Cu") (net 4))
 (via (at 158 97) (size 0.8) (drill 0.4) (layers "F.Cu" "B.Cu") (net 4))
 (via (at 142.4 99.2) (size 0.8) (drill 0.4) (layers "F.Cu" "B.Cu") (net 4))
 (segment (start 155.505 102.625) (end 155.405 102.725) (width 0.25) (layer "F.Cu") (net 8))
 (segment (start 157.1 102.625) (end 155.505 102.625) (width 0.25) (layer "F.Cu") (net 8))
 (segment (start 145.095 102.675) (end 141.2 102.675) (width 0.25) (layer "F.Cu") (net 7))
 (segment (start 141.2 102.675) (end 139.8 101.275) (width 0.25) (layer "F.Cu") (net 7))
 (segment (start 139.8 101.275) (end 137.2 101.275) (width 0.25) (layer "F.Cu") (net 7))
 (segment (start 139.8 101.275) (end 139.8 99.325) (width 0.25) (layer "F.Cu") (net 7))
 (segment (start 139.8 99.325) (end 139.825 99.3) (width 0.25) (layer "F.Cu") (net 7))
 (segment (start 154.135 97.851751) (end 154.135 97.575) (width 0.25) (layer "F.Cu") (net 2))
 (segment (start 157.783249 101.5) (end 154.135 97.851751) (width 0.25) (layer "F.Cu") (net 2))
 (segment (start 159.67 101.5) (end 157.783249 101.5) (width 0.25) (layer "F.Cu") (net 2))
 (segment (start 159.67 99.5) (end 157.33 99.5) (width 0.25) (layer "F.Cu") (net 3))
 (segment (start 157.33 99.5) (end 155.405 97.575) (width 0.25) (layer "F.Cu") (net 3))
 (segment (start 136.4 100.857538) (end 138.782038 98.4755) (width 0.25) (layer "F.Cu") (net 6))
 (segment (start 143.812251 98.4755) (end 147.635 102.298249) (width 0.25) (layer "F.Cu") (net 6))
 (segment (start 147.635 102.298249) (end 147.635 102.675) (width 0.25) (layer "F.Cu") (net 6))
 (segment (start 136.4 102.125) (end 136.4 100.857538) (width 0.25) (layer "F.Cu") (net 6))
 (segment (start 137.2 102.925) (end 137.275 103) (width 0.25) (layer "F.Cu") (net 6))
 (segment (start 137.2 102.925) (end 136.4 102.125) (width 0.25) (layer "F.Cu") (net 6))
 (segment (start 138.782038 98.4755) (end 143.812251 98.4755) (width 0.25) (layer "F.Cu") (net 6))
 (segment (start 137.275 103) (end 137.275 105.5) (width 0.25) (layer "F.Cu") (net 6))
 (segment (start 140.85 103.975) (end 145.441751 103.975) (width 0.25) (layer "F.Cu") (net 12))
 (segment (start 139.8 102.925) (end 140.85 103.975) (width 0.25) (layer "F.Cu") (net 12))
 (segment (start 146.365 103.051751) (end 146.365 102.675) (width 0.25) (layer "F.Cu") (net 12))
 (segment (start 145.441751 103.975) (end 146.365 103.051751) (width 0.25) (layer "F.Cu") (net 12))
 (segment (start 139.8 102.925) (end 139.815 102.94) (width 0.25) (layer "F.Cu") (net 12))
 (segment (start 139.815 102.94) (end 139.815 105.5) (width 0.25) (layer "F.Cu") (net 12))
 (segment (start 152.865 102.448249) (end 152.865 102.725) (width 0.25) (layer "F.Cu") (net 10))
 (segment (start 145.095 97.725) (end 145.4 98.406751) (width 0.25) (layer "F.Cu") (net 10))
 (segment (start 145.4 98.03) (end 145.095 97.725) (width 0.25) (layer "F.Cu") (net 10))
 (segment (start 148.581147 99.279059) (end 149.69581 99.279059) (width 0.25) (layer "F.Cu") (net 10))
 (segment (start 145.095 97.725) (end 145.095 98.495) (width 0.25) (layer "F.Cu") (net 10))
 (segment (start 145.4 98.406751) (end 145.4 98.03) (width 0.25) (layer "F.Cu") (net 10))
 (segment (start 145.095 98.495) (end 145.8 99.2) (width 0.25) (layer "F.Cu") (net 10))
 (segment (start 149.69581 99.279059) (end 152.865 102.448249) (width 0.25) (layer "F.Cu") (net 10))
 (via (at 145.8 99.2) (size 0.8) (drill 0.4) (layers "F.Cu" "B.Cu") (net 10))
 (via (at 148.581147 99.279059) (size 0.8) (drill 0.4) (layers "F.Cu" "B.Cu") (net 10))
 (segment (start 145.879059 99.279059) (end 148.581147 99.279059) (width 0.25) (layer "B.Cu") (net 10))
 (segment (start 145.8 99.2) (end 145.879059 99.279059) (width 0.25) (layer "B.Cu") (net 10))
 (segment (start 154.135 102.448249) (end 149.411751 97.725) (width 0.25) (layer "F.Cu") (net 11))
 (segment (start 149.411751 97.725) (end 148.905 97.725) (width 0.25) (layer "F.Cu") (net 11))
 (segment (start 154.135 102.725) (end 154.135 102.448249) (width 0.25) (layer "F.Cu") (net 11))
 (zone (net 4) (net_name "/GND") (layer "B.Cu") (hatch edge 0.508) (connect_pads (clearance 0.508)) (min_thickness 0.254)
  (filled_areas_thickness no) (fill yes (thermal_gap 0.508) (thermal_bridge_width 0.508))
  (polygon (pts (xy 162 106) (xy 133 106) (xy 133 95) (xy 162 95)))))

